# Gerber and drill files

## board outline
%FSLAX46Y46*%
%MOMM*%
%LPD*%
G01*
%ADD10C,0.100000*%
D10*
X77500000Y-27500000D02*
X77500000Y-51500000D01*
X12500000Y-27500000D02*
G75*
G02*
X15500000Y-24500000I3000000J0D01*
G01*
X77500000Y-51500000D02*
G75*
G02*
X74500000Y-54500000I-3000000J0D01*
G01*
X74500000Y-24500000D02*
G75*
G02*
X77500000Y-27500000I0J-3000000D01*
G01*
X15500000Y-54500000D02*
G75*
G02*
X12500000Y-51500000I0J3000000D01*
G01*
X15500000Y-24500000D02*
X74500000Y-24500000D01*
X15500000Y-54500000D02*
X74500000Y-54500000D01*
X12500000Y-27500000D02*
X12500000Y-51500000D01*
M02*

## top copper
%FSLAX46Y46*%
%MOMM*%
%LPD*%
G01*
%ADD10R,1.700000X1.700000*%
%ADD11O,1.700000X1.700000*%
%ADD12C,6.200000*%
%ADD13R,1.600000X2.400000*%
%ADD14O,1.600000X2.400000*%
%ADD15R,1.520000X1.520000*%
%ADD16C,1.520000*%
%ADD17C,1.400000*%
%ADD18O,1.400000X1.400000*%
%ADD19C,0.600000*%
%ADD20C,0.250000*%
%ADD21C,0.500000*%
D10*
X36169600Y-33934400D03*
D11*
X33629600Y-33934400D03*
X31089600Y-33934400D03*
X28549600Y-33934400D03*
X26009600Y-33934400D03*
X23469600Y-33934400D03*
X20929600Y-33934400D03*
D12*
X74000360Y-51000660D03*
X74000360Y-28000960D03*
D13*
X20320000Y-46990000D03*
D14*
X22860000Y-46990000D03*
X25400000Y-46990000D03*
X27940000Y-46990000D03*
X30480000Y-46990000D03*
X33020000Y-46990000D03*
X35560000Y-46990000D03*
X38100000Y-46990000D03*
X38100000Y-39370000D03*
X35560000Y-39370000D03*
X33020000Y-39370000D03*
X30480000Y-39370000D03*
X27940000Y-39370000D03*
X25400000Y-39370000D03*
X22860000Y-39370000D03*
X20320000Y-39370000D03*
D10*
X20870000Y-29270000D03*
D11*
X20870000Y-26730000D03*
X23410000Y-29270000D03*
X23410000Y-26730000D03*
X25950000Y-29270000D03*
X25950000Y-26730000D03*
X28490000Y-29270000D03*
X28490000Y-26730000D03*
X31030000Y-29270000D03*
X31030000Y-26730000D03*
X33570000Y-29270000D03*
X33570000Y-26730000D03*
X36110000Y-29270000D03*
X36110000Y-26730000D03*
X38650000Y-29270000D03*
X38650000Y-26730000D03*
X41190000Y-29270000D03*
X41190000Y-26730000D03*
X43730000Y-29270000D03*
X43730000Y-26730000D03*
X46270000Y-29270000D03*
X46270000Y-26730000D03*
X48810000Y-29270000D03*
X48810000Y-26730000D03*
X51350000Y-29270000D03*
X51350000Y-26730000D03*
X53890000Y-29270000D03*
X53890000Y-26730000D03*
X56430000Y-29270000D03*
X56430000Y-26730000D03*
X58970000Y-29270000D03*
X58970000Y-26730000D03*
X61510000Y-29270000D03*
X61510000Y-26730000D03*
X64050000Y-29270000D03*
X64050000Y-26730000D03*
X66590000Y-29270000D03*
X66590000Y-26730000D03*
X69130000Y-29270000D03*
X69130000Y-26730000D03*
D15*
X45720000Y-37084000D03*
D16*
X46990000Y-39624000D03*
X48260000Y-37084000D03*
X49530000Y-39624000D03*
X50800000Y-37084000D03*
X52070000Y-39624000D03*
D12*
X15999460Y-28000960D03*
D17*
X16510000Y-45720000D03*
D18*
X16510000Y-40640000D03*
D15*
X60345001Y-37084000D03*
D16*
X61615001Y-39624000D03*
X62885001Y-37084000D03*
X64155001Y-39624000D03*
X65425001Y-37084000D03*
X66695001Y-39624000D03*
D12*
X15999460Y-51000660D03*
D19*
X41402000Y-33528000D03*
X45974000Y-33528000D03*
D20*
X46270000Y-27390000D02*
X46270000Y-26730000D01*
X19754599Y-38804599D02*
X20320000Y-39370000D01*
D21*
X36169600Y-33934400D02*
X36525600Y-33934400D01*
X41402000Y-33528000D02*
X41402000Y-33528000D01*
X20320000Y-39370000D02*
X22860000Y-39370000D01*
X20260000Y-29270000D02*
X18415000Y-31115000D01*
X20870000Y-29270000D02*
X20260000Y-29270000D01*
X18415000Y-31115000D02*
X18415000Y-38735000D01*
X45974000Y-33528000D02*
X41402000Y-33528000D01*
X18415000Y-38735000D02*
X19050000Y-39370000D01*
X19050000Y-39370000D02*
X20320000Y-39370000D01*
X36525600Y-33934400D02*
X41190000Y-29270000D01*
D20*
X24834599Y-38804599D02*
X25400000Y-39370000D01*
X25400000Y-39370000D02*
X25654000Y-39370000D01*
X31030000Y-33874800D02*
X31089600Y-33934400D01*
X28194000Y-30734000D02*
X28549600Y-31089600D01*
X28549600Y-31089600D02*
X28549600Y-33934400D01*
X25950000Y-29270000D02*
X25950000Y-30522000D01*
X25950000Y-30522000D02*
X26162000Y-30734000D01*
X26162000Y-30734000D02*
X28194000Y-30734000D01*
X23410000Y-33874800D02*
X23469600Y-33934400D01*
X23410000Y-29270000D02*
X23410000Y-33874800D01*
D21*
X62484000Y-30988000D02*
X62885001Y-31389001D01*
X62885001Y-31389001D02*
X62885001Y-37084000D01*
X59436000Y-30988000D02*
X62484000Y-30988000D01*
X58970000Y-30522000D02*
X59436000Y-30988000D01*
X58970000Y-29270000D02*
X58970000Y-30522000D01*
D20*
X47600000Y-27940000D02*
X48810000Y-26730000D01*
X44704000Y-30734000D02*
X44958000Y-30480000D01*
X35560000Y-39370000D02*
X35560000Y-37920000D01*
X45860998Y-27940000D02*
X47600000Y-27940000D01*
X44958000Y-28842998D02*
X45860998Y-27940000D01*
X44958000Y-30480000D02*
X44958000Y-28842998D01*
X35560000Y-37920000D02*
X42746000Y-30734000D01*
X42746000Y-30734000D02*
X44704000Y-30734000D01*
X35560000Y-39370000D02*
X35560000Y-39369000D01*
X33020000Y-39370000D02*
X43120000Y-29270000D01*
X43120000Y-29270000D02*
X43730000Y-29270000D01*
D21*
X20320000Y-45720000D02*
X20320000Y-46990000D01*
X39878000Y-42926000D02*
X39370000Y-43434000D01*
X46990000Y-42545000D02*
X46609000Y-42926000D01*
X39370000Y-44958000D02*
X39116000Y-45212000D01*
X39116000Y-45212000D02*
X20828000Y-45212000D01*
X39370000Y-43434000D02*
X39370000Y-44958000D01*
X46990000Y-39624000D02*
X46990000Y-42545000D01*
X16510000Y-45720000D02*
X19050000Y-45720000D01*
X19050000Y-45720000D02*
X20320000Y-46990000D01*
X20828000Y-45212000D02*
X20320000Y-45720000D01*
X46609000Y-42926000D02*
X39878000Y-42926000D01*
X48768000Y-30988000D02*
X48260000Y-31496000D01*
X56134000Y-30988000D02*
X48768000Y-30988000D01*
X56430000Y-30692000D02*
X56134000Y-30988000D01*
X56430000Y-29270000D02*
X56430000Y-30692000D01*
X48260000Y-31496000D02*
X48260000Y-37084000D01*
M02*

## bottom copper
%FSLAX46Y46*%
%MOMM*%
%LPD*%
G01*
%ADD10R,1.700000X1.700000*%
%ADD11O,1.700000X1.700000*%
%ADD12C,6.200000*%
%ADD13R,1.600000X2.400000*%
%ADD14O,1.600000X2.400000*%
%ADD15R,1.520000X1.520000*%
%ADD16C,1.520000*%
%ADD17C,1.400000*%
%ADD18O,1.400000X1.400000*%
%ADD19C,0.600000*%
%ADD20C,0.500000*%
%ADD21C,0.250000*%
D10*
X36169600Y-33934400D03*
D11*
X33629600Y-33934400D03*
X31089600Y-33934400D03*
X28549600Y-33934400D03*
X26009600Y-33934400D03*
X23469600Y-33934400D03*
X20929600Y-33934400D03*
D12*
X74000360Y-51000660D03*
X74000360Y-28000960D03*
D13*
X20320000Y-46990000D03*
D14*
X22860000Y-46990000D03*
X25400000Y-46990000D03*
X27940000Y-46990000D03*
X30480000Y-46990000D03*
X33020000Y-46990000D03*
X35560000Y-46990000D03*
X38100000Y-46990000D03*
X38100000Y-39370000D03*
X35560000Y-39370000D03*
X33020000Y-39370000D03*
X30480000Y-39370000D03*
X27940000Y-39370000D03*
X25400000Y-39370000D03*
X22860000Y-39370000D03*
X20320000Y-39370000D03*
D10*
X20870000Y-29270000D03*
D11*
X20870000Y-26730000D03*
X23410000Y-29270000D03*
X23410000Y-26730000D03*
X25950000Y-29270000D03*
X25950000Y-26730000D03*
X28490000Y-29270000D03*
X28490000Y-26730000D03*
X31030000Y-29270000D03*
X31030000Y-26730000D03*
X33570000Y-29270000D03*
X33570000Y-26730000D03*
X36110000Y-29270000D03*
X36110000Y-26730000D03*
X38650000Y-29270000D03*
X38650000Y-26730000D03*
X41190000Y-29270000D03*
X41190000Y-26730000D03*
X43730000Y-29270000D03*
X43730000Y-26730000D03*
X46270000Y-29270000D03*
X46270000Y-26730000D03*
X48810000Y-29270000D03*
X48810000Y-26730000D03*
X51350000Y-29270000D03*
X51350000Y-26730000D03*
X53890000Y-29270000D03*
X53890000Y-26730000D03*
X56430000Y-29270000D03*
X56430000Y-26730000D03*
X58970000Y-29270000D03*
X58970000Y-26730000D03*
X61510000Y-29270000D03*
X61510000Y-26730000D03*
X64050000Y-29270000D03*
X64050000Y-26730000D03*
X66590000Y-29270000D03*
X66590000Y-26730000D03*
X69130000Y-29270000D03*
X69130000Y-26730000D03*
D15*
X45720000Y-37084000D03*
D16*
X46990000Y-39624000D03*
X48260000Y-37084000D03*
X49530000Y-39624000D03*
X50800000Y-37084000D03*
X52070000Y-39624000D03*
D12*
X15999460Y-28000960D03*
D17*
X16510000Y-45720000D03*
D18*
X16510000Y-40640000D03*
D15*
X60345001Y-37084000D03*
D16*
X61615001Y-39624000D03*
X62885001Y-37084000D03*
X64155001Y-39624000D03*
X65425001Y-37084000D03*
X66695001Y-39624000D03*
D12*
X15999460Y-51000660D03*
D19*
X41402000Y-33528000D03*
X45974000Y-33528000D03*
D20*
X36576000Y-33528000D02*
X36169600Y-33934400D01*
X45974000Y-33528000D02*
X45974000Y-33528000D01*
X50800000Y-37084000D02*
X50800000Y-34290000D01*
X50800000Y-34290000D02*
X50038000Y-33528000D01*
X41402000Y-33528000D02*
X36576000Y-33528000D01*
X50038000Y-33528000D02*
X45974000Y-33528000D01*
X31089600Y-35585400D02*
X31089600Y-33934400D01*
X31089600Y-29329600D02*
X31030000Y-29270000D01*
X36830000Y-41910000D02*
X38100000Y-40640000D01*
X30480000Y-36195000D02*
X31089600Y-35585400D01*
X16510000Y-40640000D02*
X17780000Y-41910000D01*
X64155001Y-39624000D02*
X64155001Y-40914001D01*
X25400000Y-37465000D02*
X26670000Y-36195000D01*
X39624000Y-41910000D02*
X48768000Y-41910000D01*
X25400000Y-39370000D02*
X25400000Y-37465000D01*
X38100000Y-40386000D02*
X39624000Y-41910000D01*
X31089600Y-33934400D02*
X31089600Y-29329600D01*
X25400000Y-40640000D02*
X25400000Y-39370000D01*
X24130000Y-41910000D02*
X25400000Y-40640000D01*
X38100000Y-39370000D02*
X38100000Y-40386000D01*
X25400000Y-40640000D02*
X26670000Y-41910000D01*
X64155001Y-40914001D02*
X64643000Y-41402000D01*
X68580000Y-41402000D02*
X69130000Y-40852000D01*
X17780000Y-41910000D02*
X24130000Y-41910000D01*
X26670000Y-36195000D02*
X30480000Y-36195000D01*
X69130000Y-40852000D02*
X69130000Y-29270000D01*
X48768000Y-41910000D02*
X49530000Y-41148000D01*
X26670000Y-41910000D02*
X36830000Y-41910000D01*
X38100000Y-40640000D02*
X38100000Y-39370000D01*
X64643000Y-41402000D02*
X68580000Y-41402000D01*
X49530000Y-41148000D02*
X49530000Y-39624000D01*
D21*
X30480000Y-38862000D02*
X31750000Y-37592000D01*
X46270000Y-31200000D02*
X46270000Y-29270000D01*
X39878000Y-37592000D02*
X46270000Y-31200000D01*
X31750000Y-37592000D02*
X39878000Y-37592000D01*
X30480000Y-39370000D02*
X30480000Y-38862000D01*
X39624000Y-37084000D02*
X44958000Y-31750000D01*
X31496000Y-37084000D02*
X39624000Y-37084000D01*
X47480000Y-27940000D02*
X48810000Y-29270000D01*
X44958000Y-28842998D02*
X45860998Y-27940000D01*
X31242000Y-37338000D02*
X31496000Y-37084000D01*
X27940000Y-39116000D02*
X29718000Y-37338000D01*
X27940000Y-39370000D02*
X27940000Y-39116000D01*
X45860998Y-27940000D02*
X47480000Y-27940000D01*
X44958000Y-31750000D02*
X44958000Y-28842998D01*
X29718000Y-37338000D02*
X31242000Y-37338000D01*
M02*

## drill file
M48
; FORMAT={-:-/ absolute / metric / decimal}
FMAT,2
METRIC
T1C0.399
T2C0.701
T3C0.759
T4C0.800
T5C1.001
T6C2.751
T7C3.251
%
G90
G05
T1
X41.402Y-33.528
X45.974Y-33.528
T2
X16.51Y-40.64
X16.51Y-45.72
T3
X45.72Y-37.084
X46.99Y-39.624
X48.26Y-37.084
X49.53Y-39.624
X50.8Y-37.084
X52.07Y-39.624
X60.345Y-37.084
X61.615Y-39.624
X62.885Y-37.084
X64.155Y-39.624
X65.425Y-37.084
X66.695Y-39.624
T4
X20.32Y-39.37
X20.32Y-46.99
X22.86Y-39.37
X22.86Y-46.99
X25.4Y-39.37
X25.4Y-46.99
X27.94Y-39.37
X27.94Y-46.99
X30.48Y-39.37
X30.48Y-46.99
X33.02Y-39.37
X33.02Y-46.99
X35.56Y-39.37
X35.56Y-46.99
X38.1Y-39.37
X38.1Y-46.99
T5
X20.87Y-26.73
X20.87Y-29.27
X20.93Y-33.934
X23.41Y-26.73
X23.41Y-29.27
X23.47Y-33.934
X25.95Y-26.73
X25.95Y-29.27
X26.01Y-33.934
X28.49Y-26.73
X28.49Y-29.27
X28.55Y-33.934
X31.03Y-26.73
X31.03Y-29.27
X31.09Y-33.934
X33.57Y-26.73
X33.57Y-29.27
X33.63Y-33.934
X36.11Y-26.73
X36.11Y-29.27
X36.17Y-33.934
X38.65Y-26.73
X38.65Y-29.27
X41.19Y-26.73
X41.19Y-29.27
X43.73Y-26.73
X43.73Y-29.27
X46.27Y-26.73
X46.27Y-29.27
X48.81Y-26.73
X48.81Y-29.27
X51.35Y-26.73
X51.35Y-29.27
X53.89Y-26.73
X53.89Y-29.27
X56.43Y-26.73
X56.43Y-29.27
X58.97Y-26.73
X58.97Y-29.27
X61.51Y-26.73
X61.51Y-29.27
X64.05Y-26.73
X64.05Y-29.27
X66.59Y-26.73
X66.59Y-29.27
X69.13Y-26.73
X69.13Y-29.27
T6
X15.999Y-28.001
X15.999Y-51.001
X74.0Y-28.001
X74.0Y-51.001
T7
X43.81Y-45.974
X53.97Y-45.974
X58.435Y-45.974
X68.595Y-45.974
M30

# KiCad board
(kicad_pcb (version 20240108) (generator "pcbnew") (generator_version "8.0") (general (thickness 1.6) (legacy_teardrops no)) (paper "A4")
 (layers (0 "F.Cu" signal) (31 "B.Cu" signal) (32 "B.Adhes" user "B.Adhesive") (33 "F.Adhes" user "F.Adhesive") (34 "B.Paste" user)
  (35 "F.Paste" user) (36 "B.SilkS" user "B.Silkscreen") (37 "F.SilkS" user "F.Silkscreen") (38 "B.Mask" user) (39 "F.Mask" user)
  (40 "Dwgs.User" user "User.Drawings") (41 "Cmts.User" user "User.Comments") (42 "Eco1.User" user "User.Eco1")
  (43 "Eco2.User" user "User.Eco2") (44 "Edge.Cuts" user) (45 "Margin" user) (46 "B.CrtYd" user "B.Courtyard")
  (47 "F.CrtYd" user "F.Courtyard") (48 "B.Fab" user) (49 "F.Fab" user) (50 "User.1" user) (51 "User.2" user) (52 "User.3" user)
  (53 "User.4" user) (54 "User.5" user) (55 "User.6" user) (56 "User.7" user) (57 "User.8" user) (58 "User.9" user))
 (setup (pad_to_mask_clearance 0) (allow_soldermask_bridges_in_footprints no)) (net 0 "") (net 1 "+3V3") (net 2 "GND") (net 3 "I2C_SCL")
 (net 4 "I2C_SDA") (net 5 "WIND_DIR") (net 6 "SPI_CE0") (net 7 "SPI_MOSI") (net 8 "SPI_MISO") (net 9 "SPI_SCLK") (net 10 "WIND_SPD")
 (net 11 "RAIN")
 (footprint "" (layer "F.Cu") (at 53.96992 45.974)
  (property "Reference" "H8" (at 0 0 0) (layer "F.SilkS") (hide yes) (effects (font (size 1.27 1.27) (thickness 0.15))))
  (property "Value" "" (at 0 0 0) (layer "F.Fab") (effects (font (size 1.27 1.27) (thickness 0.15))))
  (pad "" np_thru_hole circle (at 0 0) (size 3.25 3.25) (drill 3.2512) (layers "F&B.Cu" "*.Mask")))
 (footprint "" (layer "F.Cu") (at 28.5496 33.9344)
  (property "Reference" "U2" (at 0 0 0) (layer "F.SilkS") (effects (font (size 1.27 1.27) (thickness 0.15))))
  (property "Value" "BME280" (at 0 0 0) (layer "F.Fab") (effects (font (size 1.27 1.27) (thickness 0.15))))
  (pad "1" thru_hole rect (at 7.62 0) (size 1.7 1.7) (drill 1.00076) (layers "*.Cu" "*.Mask") (remove_unused_layers no) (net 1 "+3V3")
   (thermal_bridge_angle 45))
  (pad "2" thru_hole oval (at 5.08 0) (size 1.7 1.7) (drill 1.00076) (layers "*.Cu" "*.Mask") (remove_unused_layers no)
   (thermal_bridge_angle 45))
  (pad "3" thru_hole oval (at 2.54 0) (size 1.7 1.7) (drill 1.00076) (layers "*.Cu" "*.Mask") (remove_unused_layers no) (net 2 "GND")
   (thermal_bridge_angle 45))
  (pad "4" thru_hole oval (at 0 0) (size 1.7 1.7) (drill 1.00076) (layers "*.Cu" "*.Mask") (remove_unused_layers no) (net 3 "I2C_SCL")
   (thermal_bridge_angle 45))
  (pad "5" thru_hole oval (at -2.54 0) (size 1.7 1.7) (drill 1.00076) (layers "*.Cu" "*.Mask") (remove_unused_layers no)
   (thermal_bridge_angle 45))
  (pad "6" thru_hole oval (at -5.08 0) (size 1.7 1.7) (drill 1.00076) (layers "*.Cu" "*.Mask") (remove_unused_layers no) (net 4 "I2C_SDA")
   (thermal_bridge_angle 45))
  (pad "7" thru_hole oval (at -7.62 0) (size 1.7 1.7) (drill 1.00076) (layers "*.Cu" "*.Mask") (remove_unused_layers no)
   (thermal_bridge_angle 45)))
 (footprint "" (layer "F.Cu") (at 43.80992 45.974)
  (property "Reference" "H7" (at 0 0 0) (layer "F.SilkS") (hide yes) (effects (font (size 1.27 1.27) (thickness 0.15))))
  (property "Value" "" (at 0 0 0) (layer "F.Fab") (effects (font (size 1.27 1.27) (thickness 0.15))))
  (pad "" np_thru_hole circle (at 0 0) (size 3.25 3.25) (drill 3.2512) (layers "F&B.Cu" "*.Mask")))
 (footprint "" (layer "F.Cu") (at 74.00036 51.00066)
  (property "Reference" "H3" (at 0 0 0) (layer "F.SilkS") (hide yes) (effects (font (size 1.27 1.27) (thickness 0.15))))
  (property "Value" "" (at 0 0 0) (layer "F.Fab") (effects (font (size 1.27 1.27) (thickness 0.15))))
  (pad "" np_thru_hole circle (at 0 0) (size 6.2 6.2) (drill 2.75082) (layers "F&B.Cu" "*.Mask")))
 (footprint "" (layer "F.Cu") (at 74.00036 28.00096)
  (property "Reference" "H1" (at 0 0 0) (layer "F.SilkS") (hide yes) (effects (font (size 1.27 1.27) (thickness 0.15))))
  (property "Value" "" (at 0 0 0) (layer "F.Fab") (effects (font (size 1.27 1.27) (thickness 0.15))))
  (pad "" np_thru_hole circle (at 0 0) (size 6.2 6.2) (drill 2.75082) (layers "F&B.Cu" "*.Mask")))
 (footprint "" (layer "F.Cu") (at 68.59524 45.974)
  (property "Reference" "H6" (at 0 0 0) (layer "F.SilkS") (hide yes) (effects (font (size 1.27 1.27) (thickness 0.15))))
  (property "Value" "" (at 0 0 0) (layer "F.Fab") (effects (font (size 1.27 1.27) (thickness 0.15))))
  (pad "" np_thru_hole circle (at 0 0) (size 3.25 3.25) (drill 3.2512) (layers "F&B.Cu" "*.Mask")))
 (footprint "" (layer "F.Cu") (at 29.21 43.18)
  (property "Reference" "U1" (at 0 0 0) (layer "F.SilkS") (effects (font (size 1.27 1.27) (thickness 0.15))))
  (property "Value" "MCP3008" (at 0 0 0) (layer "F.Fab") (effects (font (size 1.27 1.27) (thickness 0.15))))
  (pad "1" thru_hole rect (at -8.89 3.81) (size 1.6 2.4) (drill 0.8001) (layers "*.Cu" "*.Mask") (remove_unused_layers no)
   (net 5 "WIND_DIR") (thermal_bridge_angle 45))
  (pad "2" thru_hole oval (at -6.35 3.81) (size 1.6 2.4) (drill 0.8001) (layers "*.Cu" "*.Mask") (remove_unused_layers no)
   (thermal_bridge_angle 45))
  (pad "3" thru_hole oval (at -3.81 3.81) (size 1.6 2.4) (drill 0.8001) (layers "*.Cu" "*.Mask") (remove_unused_layers no)
   (thermal_bridge_angle 45))
  (pad "4" thru_hole oval (at -1.27 3.81) (size 1.6 2.4) (drill 0.8001) (layers "*.Cu" "*.Mask") (remove_unused_layers no)
   (thermal_bridge_angle 45))
  (pad "5" thru_hole oval (at 1.27 3.81) (size 1.6 2.4) (drill 0.8001) (layers "*.Cu" "*.Mask") (remove_unused_layers no)
   (thermal_bridge_angle 45))
  (pad "6" thru_hole oval (at 3.81 3.81) (size 1.6 2.4) (drill 0.8001) (layers "*.Cu" "*.Mask") (remove_unused_layers no)
   (thermal_bridge_angle 45))
  (pad "7" thru_hole oval (at 6.35 3.81) (size 1.6 2.4) (drill 0.8001) (layers "*.Cu" "*.Mask") (remove_unused_layers no)
   (thermal_bridge_angle 45))
  (pad "8" thru_hole oval (at 8.89 3.81) (size 1.6 2.4) (drill 0.8001) (layers "*.Cu" "*.Mask") (remove_unused_layers no)
   (thermal_bridge_angle 45))
  (pad "9" thru_hole oval (at 8.89 -3.81) (size 1.6 2.4) (drill 0.8001) (layers "*.Cu" "*.Mask") (remove_unused_layers no) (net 2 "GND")
   (thermal_bridge_angle 45))
  (pad "10" thru_hole oval (at 6.35 -3.81) (size 1.6 2.4) (drill 0.8001) (layers "*.Cu" "*.Mask") (remove_unused_layers no)
   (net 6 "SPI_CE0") (thermal_bridge_angle 45))
  (pad "11" thru_hole oval (at 3.81 -3.81) (size 1.6 2.4) (drill 0.8001) (layers "*.Cu" "*.Mask") (remove_unused_layers no)
   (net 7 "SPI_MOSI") (thermal_bridge_angle 45))
  (pad "12" thru_hole oval (at 1.27 -3.81) (size 1.6 2.4) (drill 0.8001) (layers "*.Cu" "*.Mask") (remove_unused_layers no)
   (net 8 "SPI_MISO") (thermal_bridge_angle 45))
  (pad "13" thru_hole oval (at -1.27 -3.81) (size 1.6 2.4) (drill 0.8001) (layers "*.Cu" "*.Mask") (remove_unused_layers no)
   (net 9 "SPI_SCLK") (thermal_bridge_angle 45))
  (pad "14" thru_hole oval (at -3.81 -3.81) (size 1.6 2.4) (drill 0.8001) (layers "*.Cu" "*.Mask") (remove_unused_layers no) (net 2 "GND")
   (thermal_bridge_angle 45))
  (pad "15" thru_hole oval (at -6.35 -3.81) (size 1.6 2.4) (drill 0.8001) (layers "*.Cu" "*.Mask") (remove_unused_layers no) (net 1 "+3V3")
   (thermal_bridge_angle 45))
  (pad "16" thru_hole oval (at -8.89 -3.81) (size 1.6 2.4) (drill 0.8001) (layers "*.Cu" "*.Mask") (remove_unused_layers no) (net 1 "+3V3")
   (thermal_bridge_angle 45)))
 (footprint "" (layer "F.Cu") (at 45 28)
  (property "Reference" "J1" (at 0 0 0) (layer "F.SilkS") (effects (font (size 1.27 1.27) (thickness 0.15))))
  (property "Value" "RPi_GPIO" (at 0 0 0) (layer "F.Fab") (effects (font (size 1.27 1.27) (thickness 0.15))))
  (pad "1" thru_hole rect (at -24.13 1.27) (size 1.7 1.7) (drill 1.00076) (layers "*.Cu" "*.Mask") (remove_unused_layers no) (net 1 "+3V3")
   (thermal_bridge_angle 45))
  (pad "2" thru_hole oval (at -24.13 -1.27) (size 1.7 1.7) (drill 1.00076) (layers "*.Cu" "*.Mask") (remove_unused_layers no)
   (thermal_bridge_angle 45))
  (pad "3" thru_hole oval (at -21.59 1.27) (size 1.7 1.7) (drill 1.00076) (layers "*.Cu" "*.Mask") (remove_unused_layers no)
   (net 4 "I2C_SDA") (thermal_bridge_angle 45))
  (pad "4" thru_hole oval (at -21.59 -1.27) (size 1.7 1.7) (drill 1.00076) (layers "*.Cu" "*.Mask") (remove_unused_layers no)
   (thermal_bridge_angle 45))
  (pad "5" thru_hole oval (at -19.05 1.27) (size 1.7 1.7) (drill 1.00076) (layers "*.Cu" "*.Mask") (remove_unused_layers no)
   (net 3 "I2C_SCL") (thermal_bridge_angle 45))
  (pad "6" thru_hole oval (at -19.05 -1.27) (size 1.7 1.7) (drill 1.00076) (layers "*.Cu" "*.Mask") (remove_unused_layers no)
   (thermal_bridge_angle 45))
  (pad "7" thru_hole oval (at -16.51 1.27) (size 1.7 1.7) (drill 1.00076) (layers "*.Cu" "*.Mask") (remove_unused_layers no)
   (thermal_bridge_angle 45))
  (pad "8" thru_hole oval (at -16.51 -1.27) (size 1.7 1.7) (drill 1.00076) (layers "*.Cu" "*.Mask") (remove_unused_layers no)
   (thermal_bridge_angle 45))
  (pad "9" thru_hole oval (at -13.97 1.27) (size 1.7 1.7) (drill 1.00076) (layers "*.Cu" "*.Mask") (remove_unused_layers no) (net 2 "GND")
   (thermal_bridge_angle 45))
  (pad "10" thru_hole oval (at -13.97 -1.27) (size 1.7 1.7) (drill 1.00076) (layers "*.Cu" "*.Mask") (remove_unused_layers no)
   (thermal_bridge_angle 45))
  (pad "11" thru_hole oval (at -11.43 1.27) (size 1.7 1.7) (drill 1.00076) (layers "*.Cu" "*.Mask") (remove_unused_layers no)
   (thermal_bridge_angle 45))
  (pad "12" thru_hole oval (at -11.43 -1.27) (size 1.7 1.7) (drill 1.00076) (layers "*.Cu" "*.Mask") (remove_unused_layers no)
   (thermal_bridge_angle 45))
  (pad "13" thru_hole oval (at -8.89 1.27) (size 1.7 1.7) (drill 1.00076) (layers "*.Cu" "*.Mask") (remove_unused_layers no)
   (thermal_bridge_angle 45))
  (pad "14" thru_hole oval (at -8.89 -1.27) (size 1.7 1.7) (drill 1.00076) (layers "*.Cu" "*.Mask") (remove_unused_layers no)
   (thermal_bridge_angle 45))
  (pad "15" thru_hole oval (at -6.35 1.27) (size 1.7 1.7) (drill 1.00076) (layers "*.Cu" "*.Mask") (remove_unused_layers no)
   (thermal_bridge_angle 45))
  (pad "16" thru_hole oval (at -6.35 -1.27) (size 1.7 1.7) (drill 1.00076) (layers "*.Cu" "*.Mask") (remove_unused_layers no)
   (thermal_bridge_angle 45))
  (pad "17" thru_hole oval (at -3.81 1.27) (size 1.7 1.7) (drill 1.00076) (layers "*.Cu" "*.Mask") (remove_unused_layers no) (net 1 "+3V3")
   (thermal_bridge_angle 45))
  (pad "18" thru_hole oval (at -3.81 -1.27) (size 1.7 1.7) (drill 1.00076) (layers "*.Cu" "*.Mask") (remove_unused_layers no)
   (thermal_bridge_angle 45))
  (pad "19" thru_hole oval (at -1.27 1.27) (size 1.7 1.7) (drill 1.00076) (layers "*.Cu" "*.Mask") (remove_unused_layers no)
   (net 7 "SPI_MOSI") (thermal_bridge_angle 45))
  (pad "20" thru_hole oval (at -1.27 -1.27) (size 1.7 1.7) (drill 1.00076) (layers "*.Cu" "*.Mask") (remove_unused_layers no)
   (thermal_bridge_angle 45))
  (pad "21" thru_hole oval (at 1.27 1.27) (size 1.7 1.7) (drill 1.00076) (layers "*.Cu" "*.Mask") (remove_unused_layers no)
   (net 8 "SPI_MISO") (thermal_bridge_angle 45))
  (pad "22" thru_hole oval (at 1.27 -1.27) (size 1.7 1.7) (drill 1.00076) (layers "*.Cu" "*.Mask") (remove_unused_layers no)
   (thermal_bridge_angle 45))
  (pad "23" thru_hole oval (at 3.81 1.27) (size 1.7 1.7) (drill 1.00076) (layers "*.Cu" "*.Mask") (remove_unused_layers no)
   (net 9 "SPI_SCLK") (thermal_bridge_angle 45))
  (pad "24" thru_hole oval (at 3.81 -1.27) (size 1.7 1.7) (drill 1.00076) (layers "*.Cu" "*.Mask") (remove_unused_layers no)
   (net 6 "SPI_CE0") (thermal_bridge_angle 45))
  (pad "25" thru_hole oval (at 6.35 1.27) (size 1.7 1.7) (drill 1.00076) (layers "*.Cu" "*.Mask") (remove_unused_layers no)
   (thermal_bridge_angle 45))
  (pad "26" thru_hole oval (at 6.35 -1.27) (size 1.7 1.7) (drill 1.00076) (layers "*.Cu" "*.Mask") (remove_unused_layers no)
   (thermal_bridge_angle 45))
  (pad "27" thru_hole oval (at 8.89 1.27) (size 1.7 1.7) (drill 1.00076) (layers "*.Cu" "*.Mask") (remove_unused_layers no)
   (thermal_bridge_angle 45))
  (pad "28" thru_hole oval (at 8.89 -1.27) (size 1.7 1.7) (drill 1.00076) (layers "*.Cu" "*.Mask") (remove_unused_layers no)
   (thermal_bridge_angle 45))
  (pad "29" thru_hole oval (at 11.43 1.27) (size 1.7 1.7) (drill 1.00076) (layers "*.Cu" "*.Mask") (remove_unused_layers no)
   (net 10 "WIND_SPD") (thermal_bridge_angle 45))
  (pad "30" thru_hole oval (at 11.43 -1.27) (size 1.7 1.7) (drill 1.00076) (layers "*.Cu" "*.Mask") (remove_unused_layers no)
   (thermal_bridge_angle 45))
  (pad "31" thru_hole oval (at 13.97 1.27) (size 1.7 1.7) (drill 1.00076) (layers "*.Cu" "*.Mask") (remove_unused_layers no) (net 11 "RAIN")
   (thermal_bridge_angle 45))
  (pad "32" thru_hole oval (at 13.97 -1.27) (size 1.7 1.7) (drill 1.00076) (layers "*.Cu" "*.Mask") (remove_unused_layers no)
   (thermal_bridge_angle 45))
  (pad "33" thru_hole oval (at 16.51 1.27) (size 1.7 1.7) (drill 1.00076) (layers "*.Cu" "*.Mask") (remove_unused_layers no)
   (thermal_bridge_angle 45))
  (pad "34" thru_hole oval (at 16.51 -1.27) (size 1.7 1.7) (drill 1.00076) (layers "*.Cu" "*.Mask") (remove_unused_layers no)
   (thermal_bridge_angle 45))
  (pad "35" thru_hole oval (at 19.05 1.27) (size 1.7 1.7) (drill 1.00076) (layers "*.Cu" "*.Mask") (remove_unused_layers no)
   (thermal_bridge_angle 45))
  (pad "36" thru_hole oval (at 19.05 -1.27) (size 1.7 1.7) (drill 1.00076) (layers "*.Cu" "*.Mask") (remove_unused_layers no)
   (thermal_bridge_angle 45))
  (pad "37" thru_hole oval (at 21.59 1.27) (size 1.7 1.7) (drill 1.00076) (layers "*.Cu" "*.Mask") (remove_unused_layers no)
   (thermal_bridge_angle 45))
  (pad "38" thru_hole oval (at 21.59 -1.27) (size 1.7 1.7) (drill 1.00076) (layers "*.Cu" "*.Mask") (remove_unused_layers no)
   (thermal_bridge_angle 45))
  (pad "39" thru_hole oval (at 24.13 1.27) (size 1.7 1.7) (drill 1.00076) (layers "*.Cu" "*.Mask") (remove_unused_layers no) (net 2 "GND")
   (thermal_bridge_angle 45))
  (pad "40" thru_hole oval (at 24.13 -1.27) (size 1.7 1.7) (drill 1.00076) (layers "*.Cu" "*.Mask") (remove_unused_layers no)
   (thermal_bridge_angle 45)))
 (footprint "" (layer "F.Cu") (at 48.895 38.354)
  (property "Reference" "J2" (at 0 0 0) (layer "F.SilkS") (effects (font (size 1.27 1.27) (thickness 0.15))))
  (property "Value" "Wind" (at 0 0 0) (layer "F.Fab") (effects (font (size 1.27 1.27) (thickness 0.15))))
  (pad "1" thru_hole rect (at -3.175 -1.27) (size 1.52 1.52) (drill 0.75946) (layers "*.Cu" "*.Mask") (remove_unused_layers no)
   (thermal_bridge_angle 45))
  (pad "2" thru_hole circle (at -1.905 1.27) (size 1.52 1.52) (drill 0.75946) (layers "*.Cu" "*.Mask") (remove_unused_layers no)
   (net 5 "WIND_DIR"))
  (pad "3" thru_hole circle (at -0.635 -1.27) (size 1.52 1.52) (drill 0.75946) (layers "*.Cu" "*.Mask") (remove_unused_layers no)
   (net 10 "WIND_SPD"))
  (pad "4" thru_hole circle (at 0.635 1.27) (size 1.52 1.52) (drill 0.75946) (layers "*.Cu" "*.Mask") (remove_unused_layers no)
   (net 2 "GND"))
  (pad "5" thru_hole circle (at 1.905 -1.27) (size 1.52 1.52) (drill 0.75946) (layers "*.Cu" "*.Mask") (remove_unused_layers no)
   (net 1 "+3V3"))
  (pad "6" thru_hole circle (at 3.175 1.27) (size 1.52 1.52) (drill 0.75946) (layers "*.Cu" "*.Mask") (remove_unused_layers no)))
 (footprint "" (layer "F.Cu") (at 15.99946 28.00096)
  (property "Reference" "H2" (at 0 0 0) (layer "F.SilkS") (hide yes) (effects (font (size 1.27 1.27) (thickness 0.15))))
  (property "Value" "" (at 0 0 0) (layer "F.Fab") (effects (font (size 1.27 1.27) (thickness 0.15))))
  (pad "" np_thru_hole circle (at 0 0) (size 6.2 6.2) (drill 2.75082) (layers "F&B.Cu" "*.Mask")))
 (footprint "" (layer "F.Cu") (at 16.51 43.18)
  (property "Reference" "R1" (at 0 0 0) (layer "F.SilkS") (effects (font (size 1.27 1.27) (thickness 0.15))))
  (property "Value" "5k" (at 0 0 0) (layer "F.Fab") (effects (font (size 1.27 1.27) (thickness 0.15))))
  (pad "1" thru_hole circle (at 0 2.54) (size 1.4 1.4) (drill 0.70104) (layers "*.Cu" "*.Mask") (remove_unused_layers no) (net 5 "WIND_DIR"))
  (pad "2" thru_hole oval (at 0 -2.54) (size 1.4 1.4) (drill 0.70104) (layers "*.Cu" "*.Mask") (remove_unused_layers no) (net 2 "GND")
   (thermal_bridge_angle 45)))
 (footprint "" (layer "F.Cu") (at 63.520001 38.354)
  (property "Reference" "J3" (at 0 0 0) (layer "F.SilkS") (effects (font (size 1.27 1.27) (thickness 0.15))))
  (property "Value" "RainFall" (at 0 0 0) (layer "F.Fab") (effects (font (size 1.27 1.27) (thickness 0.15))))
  (pad "1" thru_hole rect (at -3.175 -1.27) (size 1.52 1.52) (drill 0.75946) (layers "*.Cu" "*.Mask") (remove_unused_layers no)
   (thermal_bridge_angle 45))
  (pad "2" thru_hole circle (at -1.905 1.27) (size 1.52 1.52) (drill 0.75946) (layers "*.Cu" "*.Mask") (remove_unused_layers no))
  (pad "3" thru_hole circle (at -0.635 -1.27) (size 1.52 1.52) (drill 0.75946) (layers "*.Cu" "*.Mask") (remove_unused_layers no)
   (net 11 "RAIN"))
  (pad "4" thru_hole circle (at 0.635 1.27) (size 1.52 1.52) (drill 0.75946) (layers "*.Cu" "*.Mask") (remove_unused_layers no)
   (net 2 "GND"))
  (pad "5" thru_hole circle (at 1.905 -1.27) (size 1.52 1.52) (drill 0.75946) (layers "*.Cu" "*.Mask") (remove_unused_layers no))
  (pad "6" thru_hole circle (at 3.175 1.27) (size 1.52 1.52) (drill 0.75946) (layers "*.Cu" "*.Mask") (remove_unused_layers no)))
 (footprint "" (layer "F.Cu") (at 15.99946 51.00066)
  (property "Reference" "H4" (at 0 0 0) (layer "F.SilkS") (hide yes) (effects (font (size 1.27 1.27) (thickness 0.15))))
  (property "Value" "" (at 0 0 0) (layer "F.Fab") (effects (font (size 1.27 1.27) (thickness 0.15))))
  (pad "" np_thru_hole circle (at 0 0) (size 6.2 6.2) (drill 2.75082) (layers "F&B.Cu" "*.Mask")))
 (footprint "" (layer "F.Cu") (at 58.43524 45.974)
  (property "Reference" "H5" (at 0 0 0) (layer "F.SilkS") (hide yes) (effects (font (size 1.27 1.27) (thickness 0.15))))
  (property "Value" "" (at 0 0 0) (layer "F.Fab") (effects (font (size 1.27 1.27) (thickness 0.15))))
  (pad "" np_thru_hole circle (at 0 0) (size 3.25 3.25) (drill 3.2512) (layers "F&B.Cu" "*.Mask")))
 (gr_line (start 77.5 27.5) (end 77.5 51.5) (stroke (width 0.1) (type default)) (layer "Edge.Cuts"))
 (gr_arc (start 12.5 27.5) (mid 13.37868 25.37868) (end 15.5 24.5) (stroke (width 0.1) (type default)) (layer "Edge.Cuts"))
 (gr_arc (start 77.5 51.5) (mid 76.62132 53.62132) (end 74.5 54.5) (stroke (width 0.1) (type default)) (layer "Edge.Cuts"))
 (gr_arc (start 74.5 24.5) (mid 76.62132 25.37868) (end 77.5 27.5) (stroke (width 0.1) (type default)) (layer "Edge.Cuts"))
 (gr_arc (start 15.5 54.5) (mid 13.37868 53.62132) (end 12.5 51.5) (stroke (width 0.1) (type default)) (layer "Edge.Cuts"))
 (gr_line (start 15.5 24.5) (end 74.5 24.5) (stroke (width 0.1) (type default)) (layer "Edge.Cuts"))
 (gr_line (start 15.5 54.5) (end 74.5 54.5) (stroke (width 0.1) (type default)) (layer "Edge.Cuts"))
 (gr_line (start 12.5 27.5) (end 12.5 51.5) (stroke (width 0.1) (type default)) (layer "Edge.Cuts"))
 (segment (start 46.27 27.39) (end 46.27 26.73) (width 0.25) (layer "F.Cu") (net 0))
 (segment (start 19.754599 38.804599) (end 20.32 39.37) (width 0.25) (layer "F.Cu") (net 1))
 (segment (start 36.1696 33.9344) (end 36.5256 33.9344) (width 0.5) (layer "F.Cu") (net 1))
 (segment (start 41.402 33.528) (end 41.402 33.528) (width 0.5) (layer "F.Cu") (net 1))
 (segment (start 20.32 39.37) (end 22.86 39.37) (width 0.5) (layer "F.Cu") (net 1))
 (segment (start 20.26 29.27) (end 18.415 31.115) (width 0.5) (layer "F.Cu") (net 1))
 (segment (start 20.87 29.27) (end 20.26 29.27) (width 0.5) (layer "F.Cu") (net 1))
 (segment (start 18.415 31.115) (end 18.415 38.735) (width 0.5) (layer "F.Cu") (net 1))
 (segment (start 45.974 33.528) (end 41.402 33.528) (width 0.5) (layer "F.Cu") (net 1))
 (segment (start 18.415 38.735) (end 19.05 39.37) (width 0.5) (layer "F.Cu") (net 1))
 (segment (start 19.05 39.37) (end 20.32 39.37) (width 0.5) (layer "F.Cu") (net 1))
 (segment (start 36.5256 33.9344) (end 41.19 29.27) (width 0.5) (layer "F.Cu") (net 1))
 (via (at 41.402 33.528) (size 0.6) (drill 0.39878) (layers "F.Cu" "B.Cu") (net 1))
 (via (at 45.974 33.528) (size 0.6) (drill 0.39878) (layers "F.Cu" "B.Cu") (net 1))
 (segment (start 36.576 33.528) (end 36.1696 33.9344) (width 0.5) (layer "B.Cu") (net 1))
 (segment (start 45.974 33.528) (end 45.974 33.528) (width 0.5) (layer "B.Cu") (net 1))
 (segment (start 50.8 37.084) (end 50.8 34.29) (width 0.5) (layer "B.Cu") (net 1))
 (segment (start 50.8 34.29) (end 50.038 33.528) (width 0.5) (layer "B.Cu") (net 1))
 (segment (start 41.402 33.528) (end 36.576 33.528) (width 0.5) (layer "B.Cu") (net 1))
 (segment (start 50.038 33.528) (end 45.974 33.528) (width 0.5) (layer "B.Cu") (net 1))
 (segment (start 24.834599 38.804599) (end 25.4 39.37) (width 0.25) (layer "F.Cu") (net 2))
 (segment (start 25.4 39.37) (end 25.654 39.37) (width 0.25) (layer "F.Cu") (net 2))
 (segment (start 31.03 33.8748) (end 31.0896 33.9344) (width 0.25) (layer "F.Cu") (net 2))
 (segment (start 31.0896 35.5854) (end 31.0896 33.9344) (width 0.5) (layer "B.Cu") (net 2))
 (segment (start 31.0896 29.3296) (end 31.03 29.27) (width 0.5) (layer "B.Cu") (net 2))
 (segment (start 36.83 41.91) (end 38.1 40.64) (width 0.5) (layer "B.Cu") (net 2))
 (segment (start 30.48 36.195) (end 31.0896 35.5854) (width 0.5) (layer "B.Cu") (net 2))
 (segment (start 16.51 40.64) (end 17.78 41.91) (width 0.5) (layer "B.Cu") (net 2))
 (segment (start 64.155001 39.624) (end 64.155001 40.914001) (width 0.5) (layer "B.Cu") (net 2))
 (segment (start 25.4 37.465) (end 26.67 36.195) (width 0.5) (layer "B.Cu") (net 2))
 (segment (start 39.624 41.91) (end 48.768 41.91) (width 0.5) (layer "B.Cu") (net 2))
 (segment (start 25.4 39.37) (end 25.4 37.465) (width 0.5) (layer "B.Cu") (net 2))
 (segment (start 38.1 40.386) (end 39.624 41.91) (width 0.5) (layer "B.Cu") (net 2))
 (segment (start 31.0896 33.9344) (end 31.0896 29.3296) (width 0.5) (layer "B.Cu") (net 2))
 (segment (start 25.4 40.64) (end 25.4 39.37) (width 0.5) (layer "B.Cu") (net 2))
 (segment (start 24.13 41.91) (end 25.4 40.64) (width 0.5) (layer "B.Cu") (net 2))
 (segment (start 38.1 39.37) (end 38.1 40.386) (width 0.5) (layer "B.Cu") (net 2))
 (segment (start 25.4 40.64) (end 26.67 41.91) (width 0.5) (layer "B.Cu") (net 2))
 (segment (start 64.155001 40.914001) (end 64.643 41.402) (width 0.5) (layer "B.Cu") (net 2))
 (segment (start 68.58 41.402) (end 69.13 40.852) (width 0.5) (layer "B.Cu") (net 2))
 (segment (start 17.78 41.91) (end 24.13 41.91) (width 0.5) (layer "B.Cu") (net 2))
 (segment (start 26.67 36.195) (end 30.48 36.195) (width 0.5) (layer "B.Cu") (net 2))
 (segment (start 69.13 40.852) (end 69.13 29.27) (width 0.5) (layer "B.Cu") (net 2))
 (segment (start 48.768 41.91) (end 49.53 41.148) (width 0.5) (layer "B.Cu") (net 2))
 (segment (start 26.67 41.91) (end 36.83 41.91) (width 0.5) (layer "B.Cu") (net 2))
 (segment (start 38.1 40.64) (end 38.1 39.37) (width 0.5) (layer "B.Cu") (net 2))
 (segment (start 64.643 41.402) (end 68.58 41.402) (width 0.5) (layer "B.Cu") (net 2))
 (segment (start 49.53 41.148) (end 49.53 39.624) (width 0.5) (layer "B.Cu") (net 2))
 (segment (start 28.194 30.734) (end 28.5496 31.0896) (width 0.25) (layer "F.Cu") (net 3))
 (segment (start 28.5496 31.0896) (end 28.5496 33.9344) (width 0.25) (layer "F.Cu") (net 3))
 (segment (start 25.95 29.27) (end 25.95 30.522) (width 0.25) (layer "F.Cu") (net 3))
 (segment (start 25.95 30.522) (end 26.162 30.734) (width 0.25) (layer "F.Cu") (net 3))
 (segment (start 26.162 30.734) (end 28.194 30.734) (width 0.25) (layer "F.Cu") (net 3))
 (segment (start 23.41 33.8748) (end 23.4696 33.9344) (width 0.25) (layer "F.Cu") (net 4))
 (segment (start 23.41 29.27) (end 23.41 33.8748) (width 0.25) (layer "F.Cu") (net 4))
 (segment (start 62.484 30.988) (end 62.885001 31.389001) (width 0.5) (layer "F.Cu") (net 11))
 (segment (start 62.885001 31.389001) (end 62.885001 37.084) (width 0.5) (layer "F.Cu") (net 11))
 (segment (start 59.436 30.988) (end 62.484 30.988) (width 0.5) (layer "F.Cu") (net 11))
 (segment (start 58.97 30.522) (end 59.436 30.988) (width 0.5) (layer "F.Cu") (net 11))
 (segment (start 58.97 29.27) (end 58.97 30.522) (width 0.5) (layer "F.Cu") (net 11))
 (segment (start 47.6 27.94) (end 48.81 26.73) (width 0.25) (layer "F.Cu") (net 6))
 (segment (start 44.704 30.734) (end 44.958 30.48) (width 0.25) (layer "F.Cu") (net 6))
 (segment (start 35.56 39.37) (end 35.56 37.92) (width 0.25) (layer "F.Cu") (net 6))
 (segment (start 45.860998 27.94) (end 47.6 27.94) (width 0.25) (layer "F.Cu") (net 6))
 (segment (start 44.958 28.842998) (end 45.860998 27.94) (width 0.25) (layer "F.Cu") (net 6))
 (segment (start 44.958 30.48) (end 44.958 28.842998) (width 0.25) (layer "F.Cu") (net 6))
 (segment (start 35.56 37.92) (end 42.746 30.734) (width 0.25) (layer "F.Cu") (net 6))
 (segment (start 42.746 30.734) (end 44.704 30.734) (width 0.25) (layer "F.Cu") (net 6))
 (segment (start 35.56 39.37) (end 35.56 39.369) (width 0.25) (layer "F.Cu") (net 6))
 (segment (start 30.48 38.862) (end 31.75 37.592) (width 0.25) (layer "B.Cu") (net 8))
 (segment (start 46.27 31.2) (end 46.27 29.27) (width 0.25) (layer "B.Cu") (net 8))
 (segment (start 39.878 37.592) (end 46.27 31.2) (width 0.25) (layer "B.Cu") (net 8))
 (segment (start 31.75 37.592) (end 39.878 37.592) (width 0.25) (layer "B.Cu") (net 8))
 (segment (start 30.48 39.37) (end 30.48 38.862) (width 0.25) (layer "B.Cu") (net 8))
 (segment (start 33.02 39.37) (end 43.12 29.27) (width 0.25) (layer "F.Cu") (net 7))
 (segment (start 43.12 29.27) (end 43.73 29.27) (width 0.25) (layer "F.Cu") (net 7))
 (segment (start 39.624 37.084) (end 44.958 31.75) (width 0.25) (layer "B.Cu") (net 9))
 (segment (start 31.496 37.084) (end 39.624 37.084) (width 0.25) (layer "B.Cu") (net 9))
 (segment (start 47.48 27.94) (end 48.81 29.27) (width 0.25) (layer "B.Cu") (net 9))
 (segment (start 44.958 28.842998) (end 45.860998 27.94) (width 0.25) (layer "B.Cu") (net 9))
 (segment (start 31.242 37.338) (end 31.496 37.084) (width 0.25) (layer "B.Cu") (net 9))
 (segment (start 27.94 39.116) (end 29.718 37.338) (width 0.25) (layer "B.Cu") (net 9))
 (segment (start 27.94 39.37) (end 27.94 39.116) (width 0.25) (layer "B.Cu") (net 9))
 (segment (start 45.860998 27.94) (end 47.48 27.94) (width 0.25) (layer "B.Cu") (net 9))
 (segment (start 44.958 31.75) (end 44.958 28.842998) (width 0.25) (layer "B.Cu") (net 9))
 (segment (start 29.718 37.338) (end 31.242 37.338) (width 0.25) (layer "B.Cu") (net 9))
 (segment (start 20.32 45.72) (end 20.32 46.99) (width 0.5) (layer "F.Cu") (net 5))
 (segment (start 39.878 42.926) (end 39.37 43.434) (width 0.5) (layer "F.Cu") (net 5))
 (segment (start 46.99 42.545) (end 46.609 42.926) (width 0.5) (layer "F.Cu") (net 5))
 (segment (start 39.37 44.958) (end 39.116 45.212) (width 0.5) (layer "F.Cu") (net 5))
 (segment (start 39.116 45.212) (end 20.828 45.212) (width 0.5) (layer "F.Cu") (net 5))
 (segment (start 39.37 43.434) (end 39.37 44.958) (width 0.5) (layer "F.Cu") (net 5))
 (segment (start 46.99 39.624) (end 46.99 42.545) (width 0.5) (layer "F.Cu") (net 5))
 (segment (start 16.51 45.72) (end 19.05 45.72) (width 0.5) (layer "F.Cu") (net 5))
 (segment (start 19.05 45.72) (end 20.32 46.99) (width 0.5) (layer "F.Cu") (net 5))
 (segment (start 20.828 45.212) (end 20.32 45.72) (width 0.5) (layer "F.Cu") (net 5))
 (segment (start 46.609 42.926) (end 39.878 42.926) (width 0.5) (layer "F.Cu") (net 5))
 (segment (start 48.768 30.988) (end 48.26 31.496) (width 0.5) (layer "F.Cu") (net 10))
 (segment (start 56.134 30.988) (end 48.768 30.988) (width 0.5) (layer "F.Cu") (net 10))
 (segment (start 56.43 30.692) (end 56.134 30.988) (width 0.5) (layer "F.Cu") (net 10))
 (segment (start 56.43 29.27) (end 56.43 30.692) (width 0.5) (layer "F.Cu") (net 10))
 (segment (start 48.26 31.496) (end 48.26 37.084) (width 0.5) (layer "F.Cu") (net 10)))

